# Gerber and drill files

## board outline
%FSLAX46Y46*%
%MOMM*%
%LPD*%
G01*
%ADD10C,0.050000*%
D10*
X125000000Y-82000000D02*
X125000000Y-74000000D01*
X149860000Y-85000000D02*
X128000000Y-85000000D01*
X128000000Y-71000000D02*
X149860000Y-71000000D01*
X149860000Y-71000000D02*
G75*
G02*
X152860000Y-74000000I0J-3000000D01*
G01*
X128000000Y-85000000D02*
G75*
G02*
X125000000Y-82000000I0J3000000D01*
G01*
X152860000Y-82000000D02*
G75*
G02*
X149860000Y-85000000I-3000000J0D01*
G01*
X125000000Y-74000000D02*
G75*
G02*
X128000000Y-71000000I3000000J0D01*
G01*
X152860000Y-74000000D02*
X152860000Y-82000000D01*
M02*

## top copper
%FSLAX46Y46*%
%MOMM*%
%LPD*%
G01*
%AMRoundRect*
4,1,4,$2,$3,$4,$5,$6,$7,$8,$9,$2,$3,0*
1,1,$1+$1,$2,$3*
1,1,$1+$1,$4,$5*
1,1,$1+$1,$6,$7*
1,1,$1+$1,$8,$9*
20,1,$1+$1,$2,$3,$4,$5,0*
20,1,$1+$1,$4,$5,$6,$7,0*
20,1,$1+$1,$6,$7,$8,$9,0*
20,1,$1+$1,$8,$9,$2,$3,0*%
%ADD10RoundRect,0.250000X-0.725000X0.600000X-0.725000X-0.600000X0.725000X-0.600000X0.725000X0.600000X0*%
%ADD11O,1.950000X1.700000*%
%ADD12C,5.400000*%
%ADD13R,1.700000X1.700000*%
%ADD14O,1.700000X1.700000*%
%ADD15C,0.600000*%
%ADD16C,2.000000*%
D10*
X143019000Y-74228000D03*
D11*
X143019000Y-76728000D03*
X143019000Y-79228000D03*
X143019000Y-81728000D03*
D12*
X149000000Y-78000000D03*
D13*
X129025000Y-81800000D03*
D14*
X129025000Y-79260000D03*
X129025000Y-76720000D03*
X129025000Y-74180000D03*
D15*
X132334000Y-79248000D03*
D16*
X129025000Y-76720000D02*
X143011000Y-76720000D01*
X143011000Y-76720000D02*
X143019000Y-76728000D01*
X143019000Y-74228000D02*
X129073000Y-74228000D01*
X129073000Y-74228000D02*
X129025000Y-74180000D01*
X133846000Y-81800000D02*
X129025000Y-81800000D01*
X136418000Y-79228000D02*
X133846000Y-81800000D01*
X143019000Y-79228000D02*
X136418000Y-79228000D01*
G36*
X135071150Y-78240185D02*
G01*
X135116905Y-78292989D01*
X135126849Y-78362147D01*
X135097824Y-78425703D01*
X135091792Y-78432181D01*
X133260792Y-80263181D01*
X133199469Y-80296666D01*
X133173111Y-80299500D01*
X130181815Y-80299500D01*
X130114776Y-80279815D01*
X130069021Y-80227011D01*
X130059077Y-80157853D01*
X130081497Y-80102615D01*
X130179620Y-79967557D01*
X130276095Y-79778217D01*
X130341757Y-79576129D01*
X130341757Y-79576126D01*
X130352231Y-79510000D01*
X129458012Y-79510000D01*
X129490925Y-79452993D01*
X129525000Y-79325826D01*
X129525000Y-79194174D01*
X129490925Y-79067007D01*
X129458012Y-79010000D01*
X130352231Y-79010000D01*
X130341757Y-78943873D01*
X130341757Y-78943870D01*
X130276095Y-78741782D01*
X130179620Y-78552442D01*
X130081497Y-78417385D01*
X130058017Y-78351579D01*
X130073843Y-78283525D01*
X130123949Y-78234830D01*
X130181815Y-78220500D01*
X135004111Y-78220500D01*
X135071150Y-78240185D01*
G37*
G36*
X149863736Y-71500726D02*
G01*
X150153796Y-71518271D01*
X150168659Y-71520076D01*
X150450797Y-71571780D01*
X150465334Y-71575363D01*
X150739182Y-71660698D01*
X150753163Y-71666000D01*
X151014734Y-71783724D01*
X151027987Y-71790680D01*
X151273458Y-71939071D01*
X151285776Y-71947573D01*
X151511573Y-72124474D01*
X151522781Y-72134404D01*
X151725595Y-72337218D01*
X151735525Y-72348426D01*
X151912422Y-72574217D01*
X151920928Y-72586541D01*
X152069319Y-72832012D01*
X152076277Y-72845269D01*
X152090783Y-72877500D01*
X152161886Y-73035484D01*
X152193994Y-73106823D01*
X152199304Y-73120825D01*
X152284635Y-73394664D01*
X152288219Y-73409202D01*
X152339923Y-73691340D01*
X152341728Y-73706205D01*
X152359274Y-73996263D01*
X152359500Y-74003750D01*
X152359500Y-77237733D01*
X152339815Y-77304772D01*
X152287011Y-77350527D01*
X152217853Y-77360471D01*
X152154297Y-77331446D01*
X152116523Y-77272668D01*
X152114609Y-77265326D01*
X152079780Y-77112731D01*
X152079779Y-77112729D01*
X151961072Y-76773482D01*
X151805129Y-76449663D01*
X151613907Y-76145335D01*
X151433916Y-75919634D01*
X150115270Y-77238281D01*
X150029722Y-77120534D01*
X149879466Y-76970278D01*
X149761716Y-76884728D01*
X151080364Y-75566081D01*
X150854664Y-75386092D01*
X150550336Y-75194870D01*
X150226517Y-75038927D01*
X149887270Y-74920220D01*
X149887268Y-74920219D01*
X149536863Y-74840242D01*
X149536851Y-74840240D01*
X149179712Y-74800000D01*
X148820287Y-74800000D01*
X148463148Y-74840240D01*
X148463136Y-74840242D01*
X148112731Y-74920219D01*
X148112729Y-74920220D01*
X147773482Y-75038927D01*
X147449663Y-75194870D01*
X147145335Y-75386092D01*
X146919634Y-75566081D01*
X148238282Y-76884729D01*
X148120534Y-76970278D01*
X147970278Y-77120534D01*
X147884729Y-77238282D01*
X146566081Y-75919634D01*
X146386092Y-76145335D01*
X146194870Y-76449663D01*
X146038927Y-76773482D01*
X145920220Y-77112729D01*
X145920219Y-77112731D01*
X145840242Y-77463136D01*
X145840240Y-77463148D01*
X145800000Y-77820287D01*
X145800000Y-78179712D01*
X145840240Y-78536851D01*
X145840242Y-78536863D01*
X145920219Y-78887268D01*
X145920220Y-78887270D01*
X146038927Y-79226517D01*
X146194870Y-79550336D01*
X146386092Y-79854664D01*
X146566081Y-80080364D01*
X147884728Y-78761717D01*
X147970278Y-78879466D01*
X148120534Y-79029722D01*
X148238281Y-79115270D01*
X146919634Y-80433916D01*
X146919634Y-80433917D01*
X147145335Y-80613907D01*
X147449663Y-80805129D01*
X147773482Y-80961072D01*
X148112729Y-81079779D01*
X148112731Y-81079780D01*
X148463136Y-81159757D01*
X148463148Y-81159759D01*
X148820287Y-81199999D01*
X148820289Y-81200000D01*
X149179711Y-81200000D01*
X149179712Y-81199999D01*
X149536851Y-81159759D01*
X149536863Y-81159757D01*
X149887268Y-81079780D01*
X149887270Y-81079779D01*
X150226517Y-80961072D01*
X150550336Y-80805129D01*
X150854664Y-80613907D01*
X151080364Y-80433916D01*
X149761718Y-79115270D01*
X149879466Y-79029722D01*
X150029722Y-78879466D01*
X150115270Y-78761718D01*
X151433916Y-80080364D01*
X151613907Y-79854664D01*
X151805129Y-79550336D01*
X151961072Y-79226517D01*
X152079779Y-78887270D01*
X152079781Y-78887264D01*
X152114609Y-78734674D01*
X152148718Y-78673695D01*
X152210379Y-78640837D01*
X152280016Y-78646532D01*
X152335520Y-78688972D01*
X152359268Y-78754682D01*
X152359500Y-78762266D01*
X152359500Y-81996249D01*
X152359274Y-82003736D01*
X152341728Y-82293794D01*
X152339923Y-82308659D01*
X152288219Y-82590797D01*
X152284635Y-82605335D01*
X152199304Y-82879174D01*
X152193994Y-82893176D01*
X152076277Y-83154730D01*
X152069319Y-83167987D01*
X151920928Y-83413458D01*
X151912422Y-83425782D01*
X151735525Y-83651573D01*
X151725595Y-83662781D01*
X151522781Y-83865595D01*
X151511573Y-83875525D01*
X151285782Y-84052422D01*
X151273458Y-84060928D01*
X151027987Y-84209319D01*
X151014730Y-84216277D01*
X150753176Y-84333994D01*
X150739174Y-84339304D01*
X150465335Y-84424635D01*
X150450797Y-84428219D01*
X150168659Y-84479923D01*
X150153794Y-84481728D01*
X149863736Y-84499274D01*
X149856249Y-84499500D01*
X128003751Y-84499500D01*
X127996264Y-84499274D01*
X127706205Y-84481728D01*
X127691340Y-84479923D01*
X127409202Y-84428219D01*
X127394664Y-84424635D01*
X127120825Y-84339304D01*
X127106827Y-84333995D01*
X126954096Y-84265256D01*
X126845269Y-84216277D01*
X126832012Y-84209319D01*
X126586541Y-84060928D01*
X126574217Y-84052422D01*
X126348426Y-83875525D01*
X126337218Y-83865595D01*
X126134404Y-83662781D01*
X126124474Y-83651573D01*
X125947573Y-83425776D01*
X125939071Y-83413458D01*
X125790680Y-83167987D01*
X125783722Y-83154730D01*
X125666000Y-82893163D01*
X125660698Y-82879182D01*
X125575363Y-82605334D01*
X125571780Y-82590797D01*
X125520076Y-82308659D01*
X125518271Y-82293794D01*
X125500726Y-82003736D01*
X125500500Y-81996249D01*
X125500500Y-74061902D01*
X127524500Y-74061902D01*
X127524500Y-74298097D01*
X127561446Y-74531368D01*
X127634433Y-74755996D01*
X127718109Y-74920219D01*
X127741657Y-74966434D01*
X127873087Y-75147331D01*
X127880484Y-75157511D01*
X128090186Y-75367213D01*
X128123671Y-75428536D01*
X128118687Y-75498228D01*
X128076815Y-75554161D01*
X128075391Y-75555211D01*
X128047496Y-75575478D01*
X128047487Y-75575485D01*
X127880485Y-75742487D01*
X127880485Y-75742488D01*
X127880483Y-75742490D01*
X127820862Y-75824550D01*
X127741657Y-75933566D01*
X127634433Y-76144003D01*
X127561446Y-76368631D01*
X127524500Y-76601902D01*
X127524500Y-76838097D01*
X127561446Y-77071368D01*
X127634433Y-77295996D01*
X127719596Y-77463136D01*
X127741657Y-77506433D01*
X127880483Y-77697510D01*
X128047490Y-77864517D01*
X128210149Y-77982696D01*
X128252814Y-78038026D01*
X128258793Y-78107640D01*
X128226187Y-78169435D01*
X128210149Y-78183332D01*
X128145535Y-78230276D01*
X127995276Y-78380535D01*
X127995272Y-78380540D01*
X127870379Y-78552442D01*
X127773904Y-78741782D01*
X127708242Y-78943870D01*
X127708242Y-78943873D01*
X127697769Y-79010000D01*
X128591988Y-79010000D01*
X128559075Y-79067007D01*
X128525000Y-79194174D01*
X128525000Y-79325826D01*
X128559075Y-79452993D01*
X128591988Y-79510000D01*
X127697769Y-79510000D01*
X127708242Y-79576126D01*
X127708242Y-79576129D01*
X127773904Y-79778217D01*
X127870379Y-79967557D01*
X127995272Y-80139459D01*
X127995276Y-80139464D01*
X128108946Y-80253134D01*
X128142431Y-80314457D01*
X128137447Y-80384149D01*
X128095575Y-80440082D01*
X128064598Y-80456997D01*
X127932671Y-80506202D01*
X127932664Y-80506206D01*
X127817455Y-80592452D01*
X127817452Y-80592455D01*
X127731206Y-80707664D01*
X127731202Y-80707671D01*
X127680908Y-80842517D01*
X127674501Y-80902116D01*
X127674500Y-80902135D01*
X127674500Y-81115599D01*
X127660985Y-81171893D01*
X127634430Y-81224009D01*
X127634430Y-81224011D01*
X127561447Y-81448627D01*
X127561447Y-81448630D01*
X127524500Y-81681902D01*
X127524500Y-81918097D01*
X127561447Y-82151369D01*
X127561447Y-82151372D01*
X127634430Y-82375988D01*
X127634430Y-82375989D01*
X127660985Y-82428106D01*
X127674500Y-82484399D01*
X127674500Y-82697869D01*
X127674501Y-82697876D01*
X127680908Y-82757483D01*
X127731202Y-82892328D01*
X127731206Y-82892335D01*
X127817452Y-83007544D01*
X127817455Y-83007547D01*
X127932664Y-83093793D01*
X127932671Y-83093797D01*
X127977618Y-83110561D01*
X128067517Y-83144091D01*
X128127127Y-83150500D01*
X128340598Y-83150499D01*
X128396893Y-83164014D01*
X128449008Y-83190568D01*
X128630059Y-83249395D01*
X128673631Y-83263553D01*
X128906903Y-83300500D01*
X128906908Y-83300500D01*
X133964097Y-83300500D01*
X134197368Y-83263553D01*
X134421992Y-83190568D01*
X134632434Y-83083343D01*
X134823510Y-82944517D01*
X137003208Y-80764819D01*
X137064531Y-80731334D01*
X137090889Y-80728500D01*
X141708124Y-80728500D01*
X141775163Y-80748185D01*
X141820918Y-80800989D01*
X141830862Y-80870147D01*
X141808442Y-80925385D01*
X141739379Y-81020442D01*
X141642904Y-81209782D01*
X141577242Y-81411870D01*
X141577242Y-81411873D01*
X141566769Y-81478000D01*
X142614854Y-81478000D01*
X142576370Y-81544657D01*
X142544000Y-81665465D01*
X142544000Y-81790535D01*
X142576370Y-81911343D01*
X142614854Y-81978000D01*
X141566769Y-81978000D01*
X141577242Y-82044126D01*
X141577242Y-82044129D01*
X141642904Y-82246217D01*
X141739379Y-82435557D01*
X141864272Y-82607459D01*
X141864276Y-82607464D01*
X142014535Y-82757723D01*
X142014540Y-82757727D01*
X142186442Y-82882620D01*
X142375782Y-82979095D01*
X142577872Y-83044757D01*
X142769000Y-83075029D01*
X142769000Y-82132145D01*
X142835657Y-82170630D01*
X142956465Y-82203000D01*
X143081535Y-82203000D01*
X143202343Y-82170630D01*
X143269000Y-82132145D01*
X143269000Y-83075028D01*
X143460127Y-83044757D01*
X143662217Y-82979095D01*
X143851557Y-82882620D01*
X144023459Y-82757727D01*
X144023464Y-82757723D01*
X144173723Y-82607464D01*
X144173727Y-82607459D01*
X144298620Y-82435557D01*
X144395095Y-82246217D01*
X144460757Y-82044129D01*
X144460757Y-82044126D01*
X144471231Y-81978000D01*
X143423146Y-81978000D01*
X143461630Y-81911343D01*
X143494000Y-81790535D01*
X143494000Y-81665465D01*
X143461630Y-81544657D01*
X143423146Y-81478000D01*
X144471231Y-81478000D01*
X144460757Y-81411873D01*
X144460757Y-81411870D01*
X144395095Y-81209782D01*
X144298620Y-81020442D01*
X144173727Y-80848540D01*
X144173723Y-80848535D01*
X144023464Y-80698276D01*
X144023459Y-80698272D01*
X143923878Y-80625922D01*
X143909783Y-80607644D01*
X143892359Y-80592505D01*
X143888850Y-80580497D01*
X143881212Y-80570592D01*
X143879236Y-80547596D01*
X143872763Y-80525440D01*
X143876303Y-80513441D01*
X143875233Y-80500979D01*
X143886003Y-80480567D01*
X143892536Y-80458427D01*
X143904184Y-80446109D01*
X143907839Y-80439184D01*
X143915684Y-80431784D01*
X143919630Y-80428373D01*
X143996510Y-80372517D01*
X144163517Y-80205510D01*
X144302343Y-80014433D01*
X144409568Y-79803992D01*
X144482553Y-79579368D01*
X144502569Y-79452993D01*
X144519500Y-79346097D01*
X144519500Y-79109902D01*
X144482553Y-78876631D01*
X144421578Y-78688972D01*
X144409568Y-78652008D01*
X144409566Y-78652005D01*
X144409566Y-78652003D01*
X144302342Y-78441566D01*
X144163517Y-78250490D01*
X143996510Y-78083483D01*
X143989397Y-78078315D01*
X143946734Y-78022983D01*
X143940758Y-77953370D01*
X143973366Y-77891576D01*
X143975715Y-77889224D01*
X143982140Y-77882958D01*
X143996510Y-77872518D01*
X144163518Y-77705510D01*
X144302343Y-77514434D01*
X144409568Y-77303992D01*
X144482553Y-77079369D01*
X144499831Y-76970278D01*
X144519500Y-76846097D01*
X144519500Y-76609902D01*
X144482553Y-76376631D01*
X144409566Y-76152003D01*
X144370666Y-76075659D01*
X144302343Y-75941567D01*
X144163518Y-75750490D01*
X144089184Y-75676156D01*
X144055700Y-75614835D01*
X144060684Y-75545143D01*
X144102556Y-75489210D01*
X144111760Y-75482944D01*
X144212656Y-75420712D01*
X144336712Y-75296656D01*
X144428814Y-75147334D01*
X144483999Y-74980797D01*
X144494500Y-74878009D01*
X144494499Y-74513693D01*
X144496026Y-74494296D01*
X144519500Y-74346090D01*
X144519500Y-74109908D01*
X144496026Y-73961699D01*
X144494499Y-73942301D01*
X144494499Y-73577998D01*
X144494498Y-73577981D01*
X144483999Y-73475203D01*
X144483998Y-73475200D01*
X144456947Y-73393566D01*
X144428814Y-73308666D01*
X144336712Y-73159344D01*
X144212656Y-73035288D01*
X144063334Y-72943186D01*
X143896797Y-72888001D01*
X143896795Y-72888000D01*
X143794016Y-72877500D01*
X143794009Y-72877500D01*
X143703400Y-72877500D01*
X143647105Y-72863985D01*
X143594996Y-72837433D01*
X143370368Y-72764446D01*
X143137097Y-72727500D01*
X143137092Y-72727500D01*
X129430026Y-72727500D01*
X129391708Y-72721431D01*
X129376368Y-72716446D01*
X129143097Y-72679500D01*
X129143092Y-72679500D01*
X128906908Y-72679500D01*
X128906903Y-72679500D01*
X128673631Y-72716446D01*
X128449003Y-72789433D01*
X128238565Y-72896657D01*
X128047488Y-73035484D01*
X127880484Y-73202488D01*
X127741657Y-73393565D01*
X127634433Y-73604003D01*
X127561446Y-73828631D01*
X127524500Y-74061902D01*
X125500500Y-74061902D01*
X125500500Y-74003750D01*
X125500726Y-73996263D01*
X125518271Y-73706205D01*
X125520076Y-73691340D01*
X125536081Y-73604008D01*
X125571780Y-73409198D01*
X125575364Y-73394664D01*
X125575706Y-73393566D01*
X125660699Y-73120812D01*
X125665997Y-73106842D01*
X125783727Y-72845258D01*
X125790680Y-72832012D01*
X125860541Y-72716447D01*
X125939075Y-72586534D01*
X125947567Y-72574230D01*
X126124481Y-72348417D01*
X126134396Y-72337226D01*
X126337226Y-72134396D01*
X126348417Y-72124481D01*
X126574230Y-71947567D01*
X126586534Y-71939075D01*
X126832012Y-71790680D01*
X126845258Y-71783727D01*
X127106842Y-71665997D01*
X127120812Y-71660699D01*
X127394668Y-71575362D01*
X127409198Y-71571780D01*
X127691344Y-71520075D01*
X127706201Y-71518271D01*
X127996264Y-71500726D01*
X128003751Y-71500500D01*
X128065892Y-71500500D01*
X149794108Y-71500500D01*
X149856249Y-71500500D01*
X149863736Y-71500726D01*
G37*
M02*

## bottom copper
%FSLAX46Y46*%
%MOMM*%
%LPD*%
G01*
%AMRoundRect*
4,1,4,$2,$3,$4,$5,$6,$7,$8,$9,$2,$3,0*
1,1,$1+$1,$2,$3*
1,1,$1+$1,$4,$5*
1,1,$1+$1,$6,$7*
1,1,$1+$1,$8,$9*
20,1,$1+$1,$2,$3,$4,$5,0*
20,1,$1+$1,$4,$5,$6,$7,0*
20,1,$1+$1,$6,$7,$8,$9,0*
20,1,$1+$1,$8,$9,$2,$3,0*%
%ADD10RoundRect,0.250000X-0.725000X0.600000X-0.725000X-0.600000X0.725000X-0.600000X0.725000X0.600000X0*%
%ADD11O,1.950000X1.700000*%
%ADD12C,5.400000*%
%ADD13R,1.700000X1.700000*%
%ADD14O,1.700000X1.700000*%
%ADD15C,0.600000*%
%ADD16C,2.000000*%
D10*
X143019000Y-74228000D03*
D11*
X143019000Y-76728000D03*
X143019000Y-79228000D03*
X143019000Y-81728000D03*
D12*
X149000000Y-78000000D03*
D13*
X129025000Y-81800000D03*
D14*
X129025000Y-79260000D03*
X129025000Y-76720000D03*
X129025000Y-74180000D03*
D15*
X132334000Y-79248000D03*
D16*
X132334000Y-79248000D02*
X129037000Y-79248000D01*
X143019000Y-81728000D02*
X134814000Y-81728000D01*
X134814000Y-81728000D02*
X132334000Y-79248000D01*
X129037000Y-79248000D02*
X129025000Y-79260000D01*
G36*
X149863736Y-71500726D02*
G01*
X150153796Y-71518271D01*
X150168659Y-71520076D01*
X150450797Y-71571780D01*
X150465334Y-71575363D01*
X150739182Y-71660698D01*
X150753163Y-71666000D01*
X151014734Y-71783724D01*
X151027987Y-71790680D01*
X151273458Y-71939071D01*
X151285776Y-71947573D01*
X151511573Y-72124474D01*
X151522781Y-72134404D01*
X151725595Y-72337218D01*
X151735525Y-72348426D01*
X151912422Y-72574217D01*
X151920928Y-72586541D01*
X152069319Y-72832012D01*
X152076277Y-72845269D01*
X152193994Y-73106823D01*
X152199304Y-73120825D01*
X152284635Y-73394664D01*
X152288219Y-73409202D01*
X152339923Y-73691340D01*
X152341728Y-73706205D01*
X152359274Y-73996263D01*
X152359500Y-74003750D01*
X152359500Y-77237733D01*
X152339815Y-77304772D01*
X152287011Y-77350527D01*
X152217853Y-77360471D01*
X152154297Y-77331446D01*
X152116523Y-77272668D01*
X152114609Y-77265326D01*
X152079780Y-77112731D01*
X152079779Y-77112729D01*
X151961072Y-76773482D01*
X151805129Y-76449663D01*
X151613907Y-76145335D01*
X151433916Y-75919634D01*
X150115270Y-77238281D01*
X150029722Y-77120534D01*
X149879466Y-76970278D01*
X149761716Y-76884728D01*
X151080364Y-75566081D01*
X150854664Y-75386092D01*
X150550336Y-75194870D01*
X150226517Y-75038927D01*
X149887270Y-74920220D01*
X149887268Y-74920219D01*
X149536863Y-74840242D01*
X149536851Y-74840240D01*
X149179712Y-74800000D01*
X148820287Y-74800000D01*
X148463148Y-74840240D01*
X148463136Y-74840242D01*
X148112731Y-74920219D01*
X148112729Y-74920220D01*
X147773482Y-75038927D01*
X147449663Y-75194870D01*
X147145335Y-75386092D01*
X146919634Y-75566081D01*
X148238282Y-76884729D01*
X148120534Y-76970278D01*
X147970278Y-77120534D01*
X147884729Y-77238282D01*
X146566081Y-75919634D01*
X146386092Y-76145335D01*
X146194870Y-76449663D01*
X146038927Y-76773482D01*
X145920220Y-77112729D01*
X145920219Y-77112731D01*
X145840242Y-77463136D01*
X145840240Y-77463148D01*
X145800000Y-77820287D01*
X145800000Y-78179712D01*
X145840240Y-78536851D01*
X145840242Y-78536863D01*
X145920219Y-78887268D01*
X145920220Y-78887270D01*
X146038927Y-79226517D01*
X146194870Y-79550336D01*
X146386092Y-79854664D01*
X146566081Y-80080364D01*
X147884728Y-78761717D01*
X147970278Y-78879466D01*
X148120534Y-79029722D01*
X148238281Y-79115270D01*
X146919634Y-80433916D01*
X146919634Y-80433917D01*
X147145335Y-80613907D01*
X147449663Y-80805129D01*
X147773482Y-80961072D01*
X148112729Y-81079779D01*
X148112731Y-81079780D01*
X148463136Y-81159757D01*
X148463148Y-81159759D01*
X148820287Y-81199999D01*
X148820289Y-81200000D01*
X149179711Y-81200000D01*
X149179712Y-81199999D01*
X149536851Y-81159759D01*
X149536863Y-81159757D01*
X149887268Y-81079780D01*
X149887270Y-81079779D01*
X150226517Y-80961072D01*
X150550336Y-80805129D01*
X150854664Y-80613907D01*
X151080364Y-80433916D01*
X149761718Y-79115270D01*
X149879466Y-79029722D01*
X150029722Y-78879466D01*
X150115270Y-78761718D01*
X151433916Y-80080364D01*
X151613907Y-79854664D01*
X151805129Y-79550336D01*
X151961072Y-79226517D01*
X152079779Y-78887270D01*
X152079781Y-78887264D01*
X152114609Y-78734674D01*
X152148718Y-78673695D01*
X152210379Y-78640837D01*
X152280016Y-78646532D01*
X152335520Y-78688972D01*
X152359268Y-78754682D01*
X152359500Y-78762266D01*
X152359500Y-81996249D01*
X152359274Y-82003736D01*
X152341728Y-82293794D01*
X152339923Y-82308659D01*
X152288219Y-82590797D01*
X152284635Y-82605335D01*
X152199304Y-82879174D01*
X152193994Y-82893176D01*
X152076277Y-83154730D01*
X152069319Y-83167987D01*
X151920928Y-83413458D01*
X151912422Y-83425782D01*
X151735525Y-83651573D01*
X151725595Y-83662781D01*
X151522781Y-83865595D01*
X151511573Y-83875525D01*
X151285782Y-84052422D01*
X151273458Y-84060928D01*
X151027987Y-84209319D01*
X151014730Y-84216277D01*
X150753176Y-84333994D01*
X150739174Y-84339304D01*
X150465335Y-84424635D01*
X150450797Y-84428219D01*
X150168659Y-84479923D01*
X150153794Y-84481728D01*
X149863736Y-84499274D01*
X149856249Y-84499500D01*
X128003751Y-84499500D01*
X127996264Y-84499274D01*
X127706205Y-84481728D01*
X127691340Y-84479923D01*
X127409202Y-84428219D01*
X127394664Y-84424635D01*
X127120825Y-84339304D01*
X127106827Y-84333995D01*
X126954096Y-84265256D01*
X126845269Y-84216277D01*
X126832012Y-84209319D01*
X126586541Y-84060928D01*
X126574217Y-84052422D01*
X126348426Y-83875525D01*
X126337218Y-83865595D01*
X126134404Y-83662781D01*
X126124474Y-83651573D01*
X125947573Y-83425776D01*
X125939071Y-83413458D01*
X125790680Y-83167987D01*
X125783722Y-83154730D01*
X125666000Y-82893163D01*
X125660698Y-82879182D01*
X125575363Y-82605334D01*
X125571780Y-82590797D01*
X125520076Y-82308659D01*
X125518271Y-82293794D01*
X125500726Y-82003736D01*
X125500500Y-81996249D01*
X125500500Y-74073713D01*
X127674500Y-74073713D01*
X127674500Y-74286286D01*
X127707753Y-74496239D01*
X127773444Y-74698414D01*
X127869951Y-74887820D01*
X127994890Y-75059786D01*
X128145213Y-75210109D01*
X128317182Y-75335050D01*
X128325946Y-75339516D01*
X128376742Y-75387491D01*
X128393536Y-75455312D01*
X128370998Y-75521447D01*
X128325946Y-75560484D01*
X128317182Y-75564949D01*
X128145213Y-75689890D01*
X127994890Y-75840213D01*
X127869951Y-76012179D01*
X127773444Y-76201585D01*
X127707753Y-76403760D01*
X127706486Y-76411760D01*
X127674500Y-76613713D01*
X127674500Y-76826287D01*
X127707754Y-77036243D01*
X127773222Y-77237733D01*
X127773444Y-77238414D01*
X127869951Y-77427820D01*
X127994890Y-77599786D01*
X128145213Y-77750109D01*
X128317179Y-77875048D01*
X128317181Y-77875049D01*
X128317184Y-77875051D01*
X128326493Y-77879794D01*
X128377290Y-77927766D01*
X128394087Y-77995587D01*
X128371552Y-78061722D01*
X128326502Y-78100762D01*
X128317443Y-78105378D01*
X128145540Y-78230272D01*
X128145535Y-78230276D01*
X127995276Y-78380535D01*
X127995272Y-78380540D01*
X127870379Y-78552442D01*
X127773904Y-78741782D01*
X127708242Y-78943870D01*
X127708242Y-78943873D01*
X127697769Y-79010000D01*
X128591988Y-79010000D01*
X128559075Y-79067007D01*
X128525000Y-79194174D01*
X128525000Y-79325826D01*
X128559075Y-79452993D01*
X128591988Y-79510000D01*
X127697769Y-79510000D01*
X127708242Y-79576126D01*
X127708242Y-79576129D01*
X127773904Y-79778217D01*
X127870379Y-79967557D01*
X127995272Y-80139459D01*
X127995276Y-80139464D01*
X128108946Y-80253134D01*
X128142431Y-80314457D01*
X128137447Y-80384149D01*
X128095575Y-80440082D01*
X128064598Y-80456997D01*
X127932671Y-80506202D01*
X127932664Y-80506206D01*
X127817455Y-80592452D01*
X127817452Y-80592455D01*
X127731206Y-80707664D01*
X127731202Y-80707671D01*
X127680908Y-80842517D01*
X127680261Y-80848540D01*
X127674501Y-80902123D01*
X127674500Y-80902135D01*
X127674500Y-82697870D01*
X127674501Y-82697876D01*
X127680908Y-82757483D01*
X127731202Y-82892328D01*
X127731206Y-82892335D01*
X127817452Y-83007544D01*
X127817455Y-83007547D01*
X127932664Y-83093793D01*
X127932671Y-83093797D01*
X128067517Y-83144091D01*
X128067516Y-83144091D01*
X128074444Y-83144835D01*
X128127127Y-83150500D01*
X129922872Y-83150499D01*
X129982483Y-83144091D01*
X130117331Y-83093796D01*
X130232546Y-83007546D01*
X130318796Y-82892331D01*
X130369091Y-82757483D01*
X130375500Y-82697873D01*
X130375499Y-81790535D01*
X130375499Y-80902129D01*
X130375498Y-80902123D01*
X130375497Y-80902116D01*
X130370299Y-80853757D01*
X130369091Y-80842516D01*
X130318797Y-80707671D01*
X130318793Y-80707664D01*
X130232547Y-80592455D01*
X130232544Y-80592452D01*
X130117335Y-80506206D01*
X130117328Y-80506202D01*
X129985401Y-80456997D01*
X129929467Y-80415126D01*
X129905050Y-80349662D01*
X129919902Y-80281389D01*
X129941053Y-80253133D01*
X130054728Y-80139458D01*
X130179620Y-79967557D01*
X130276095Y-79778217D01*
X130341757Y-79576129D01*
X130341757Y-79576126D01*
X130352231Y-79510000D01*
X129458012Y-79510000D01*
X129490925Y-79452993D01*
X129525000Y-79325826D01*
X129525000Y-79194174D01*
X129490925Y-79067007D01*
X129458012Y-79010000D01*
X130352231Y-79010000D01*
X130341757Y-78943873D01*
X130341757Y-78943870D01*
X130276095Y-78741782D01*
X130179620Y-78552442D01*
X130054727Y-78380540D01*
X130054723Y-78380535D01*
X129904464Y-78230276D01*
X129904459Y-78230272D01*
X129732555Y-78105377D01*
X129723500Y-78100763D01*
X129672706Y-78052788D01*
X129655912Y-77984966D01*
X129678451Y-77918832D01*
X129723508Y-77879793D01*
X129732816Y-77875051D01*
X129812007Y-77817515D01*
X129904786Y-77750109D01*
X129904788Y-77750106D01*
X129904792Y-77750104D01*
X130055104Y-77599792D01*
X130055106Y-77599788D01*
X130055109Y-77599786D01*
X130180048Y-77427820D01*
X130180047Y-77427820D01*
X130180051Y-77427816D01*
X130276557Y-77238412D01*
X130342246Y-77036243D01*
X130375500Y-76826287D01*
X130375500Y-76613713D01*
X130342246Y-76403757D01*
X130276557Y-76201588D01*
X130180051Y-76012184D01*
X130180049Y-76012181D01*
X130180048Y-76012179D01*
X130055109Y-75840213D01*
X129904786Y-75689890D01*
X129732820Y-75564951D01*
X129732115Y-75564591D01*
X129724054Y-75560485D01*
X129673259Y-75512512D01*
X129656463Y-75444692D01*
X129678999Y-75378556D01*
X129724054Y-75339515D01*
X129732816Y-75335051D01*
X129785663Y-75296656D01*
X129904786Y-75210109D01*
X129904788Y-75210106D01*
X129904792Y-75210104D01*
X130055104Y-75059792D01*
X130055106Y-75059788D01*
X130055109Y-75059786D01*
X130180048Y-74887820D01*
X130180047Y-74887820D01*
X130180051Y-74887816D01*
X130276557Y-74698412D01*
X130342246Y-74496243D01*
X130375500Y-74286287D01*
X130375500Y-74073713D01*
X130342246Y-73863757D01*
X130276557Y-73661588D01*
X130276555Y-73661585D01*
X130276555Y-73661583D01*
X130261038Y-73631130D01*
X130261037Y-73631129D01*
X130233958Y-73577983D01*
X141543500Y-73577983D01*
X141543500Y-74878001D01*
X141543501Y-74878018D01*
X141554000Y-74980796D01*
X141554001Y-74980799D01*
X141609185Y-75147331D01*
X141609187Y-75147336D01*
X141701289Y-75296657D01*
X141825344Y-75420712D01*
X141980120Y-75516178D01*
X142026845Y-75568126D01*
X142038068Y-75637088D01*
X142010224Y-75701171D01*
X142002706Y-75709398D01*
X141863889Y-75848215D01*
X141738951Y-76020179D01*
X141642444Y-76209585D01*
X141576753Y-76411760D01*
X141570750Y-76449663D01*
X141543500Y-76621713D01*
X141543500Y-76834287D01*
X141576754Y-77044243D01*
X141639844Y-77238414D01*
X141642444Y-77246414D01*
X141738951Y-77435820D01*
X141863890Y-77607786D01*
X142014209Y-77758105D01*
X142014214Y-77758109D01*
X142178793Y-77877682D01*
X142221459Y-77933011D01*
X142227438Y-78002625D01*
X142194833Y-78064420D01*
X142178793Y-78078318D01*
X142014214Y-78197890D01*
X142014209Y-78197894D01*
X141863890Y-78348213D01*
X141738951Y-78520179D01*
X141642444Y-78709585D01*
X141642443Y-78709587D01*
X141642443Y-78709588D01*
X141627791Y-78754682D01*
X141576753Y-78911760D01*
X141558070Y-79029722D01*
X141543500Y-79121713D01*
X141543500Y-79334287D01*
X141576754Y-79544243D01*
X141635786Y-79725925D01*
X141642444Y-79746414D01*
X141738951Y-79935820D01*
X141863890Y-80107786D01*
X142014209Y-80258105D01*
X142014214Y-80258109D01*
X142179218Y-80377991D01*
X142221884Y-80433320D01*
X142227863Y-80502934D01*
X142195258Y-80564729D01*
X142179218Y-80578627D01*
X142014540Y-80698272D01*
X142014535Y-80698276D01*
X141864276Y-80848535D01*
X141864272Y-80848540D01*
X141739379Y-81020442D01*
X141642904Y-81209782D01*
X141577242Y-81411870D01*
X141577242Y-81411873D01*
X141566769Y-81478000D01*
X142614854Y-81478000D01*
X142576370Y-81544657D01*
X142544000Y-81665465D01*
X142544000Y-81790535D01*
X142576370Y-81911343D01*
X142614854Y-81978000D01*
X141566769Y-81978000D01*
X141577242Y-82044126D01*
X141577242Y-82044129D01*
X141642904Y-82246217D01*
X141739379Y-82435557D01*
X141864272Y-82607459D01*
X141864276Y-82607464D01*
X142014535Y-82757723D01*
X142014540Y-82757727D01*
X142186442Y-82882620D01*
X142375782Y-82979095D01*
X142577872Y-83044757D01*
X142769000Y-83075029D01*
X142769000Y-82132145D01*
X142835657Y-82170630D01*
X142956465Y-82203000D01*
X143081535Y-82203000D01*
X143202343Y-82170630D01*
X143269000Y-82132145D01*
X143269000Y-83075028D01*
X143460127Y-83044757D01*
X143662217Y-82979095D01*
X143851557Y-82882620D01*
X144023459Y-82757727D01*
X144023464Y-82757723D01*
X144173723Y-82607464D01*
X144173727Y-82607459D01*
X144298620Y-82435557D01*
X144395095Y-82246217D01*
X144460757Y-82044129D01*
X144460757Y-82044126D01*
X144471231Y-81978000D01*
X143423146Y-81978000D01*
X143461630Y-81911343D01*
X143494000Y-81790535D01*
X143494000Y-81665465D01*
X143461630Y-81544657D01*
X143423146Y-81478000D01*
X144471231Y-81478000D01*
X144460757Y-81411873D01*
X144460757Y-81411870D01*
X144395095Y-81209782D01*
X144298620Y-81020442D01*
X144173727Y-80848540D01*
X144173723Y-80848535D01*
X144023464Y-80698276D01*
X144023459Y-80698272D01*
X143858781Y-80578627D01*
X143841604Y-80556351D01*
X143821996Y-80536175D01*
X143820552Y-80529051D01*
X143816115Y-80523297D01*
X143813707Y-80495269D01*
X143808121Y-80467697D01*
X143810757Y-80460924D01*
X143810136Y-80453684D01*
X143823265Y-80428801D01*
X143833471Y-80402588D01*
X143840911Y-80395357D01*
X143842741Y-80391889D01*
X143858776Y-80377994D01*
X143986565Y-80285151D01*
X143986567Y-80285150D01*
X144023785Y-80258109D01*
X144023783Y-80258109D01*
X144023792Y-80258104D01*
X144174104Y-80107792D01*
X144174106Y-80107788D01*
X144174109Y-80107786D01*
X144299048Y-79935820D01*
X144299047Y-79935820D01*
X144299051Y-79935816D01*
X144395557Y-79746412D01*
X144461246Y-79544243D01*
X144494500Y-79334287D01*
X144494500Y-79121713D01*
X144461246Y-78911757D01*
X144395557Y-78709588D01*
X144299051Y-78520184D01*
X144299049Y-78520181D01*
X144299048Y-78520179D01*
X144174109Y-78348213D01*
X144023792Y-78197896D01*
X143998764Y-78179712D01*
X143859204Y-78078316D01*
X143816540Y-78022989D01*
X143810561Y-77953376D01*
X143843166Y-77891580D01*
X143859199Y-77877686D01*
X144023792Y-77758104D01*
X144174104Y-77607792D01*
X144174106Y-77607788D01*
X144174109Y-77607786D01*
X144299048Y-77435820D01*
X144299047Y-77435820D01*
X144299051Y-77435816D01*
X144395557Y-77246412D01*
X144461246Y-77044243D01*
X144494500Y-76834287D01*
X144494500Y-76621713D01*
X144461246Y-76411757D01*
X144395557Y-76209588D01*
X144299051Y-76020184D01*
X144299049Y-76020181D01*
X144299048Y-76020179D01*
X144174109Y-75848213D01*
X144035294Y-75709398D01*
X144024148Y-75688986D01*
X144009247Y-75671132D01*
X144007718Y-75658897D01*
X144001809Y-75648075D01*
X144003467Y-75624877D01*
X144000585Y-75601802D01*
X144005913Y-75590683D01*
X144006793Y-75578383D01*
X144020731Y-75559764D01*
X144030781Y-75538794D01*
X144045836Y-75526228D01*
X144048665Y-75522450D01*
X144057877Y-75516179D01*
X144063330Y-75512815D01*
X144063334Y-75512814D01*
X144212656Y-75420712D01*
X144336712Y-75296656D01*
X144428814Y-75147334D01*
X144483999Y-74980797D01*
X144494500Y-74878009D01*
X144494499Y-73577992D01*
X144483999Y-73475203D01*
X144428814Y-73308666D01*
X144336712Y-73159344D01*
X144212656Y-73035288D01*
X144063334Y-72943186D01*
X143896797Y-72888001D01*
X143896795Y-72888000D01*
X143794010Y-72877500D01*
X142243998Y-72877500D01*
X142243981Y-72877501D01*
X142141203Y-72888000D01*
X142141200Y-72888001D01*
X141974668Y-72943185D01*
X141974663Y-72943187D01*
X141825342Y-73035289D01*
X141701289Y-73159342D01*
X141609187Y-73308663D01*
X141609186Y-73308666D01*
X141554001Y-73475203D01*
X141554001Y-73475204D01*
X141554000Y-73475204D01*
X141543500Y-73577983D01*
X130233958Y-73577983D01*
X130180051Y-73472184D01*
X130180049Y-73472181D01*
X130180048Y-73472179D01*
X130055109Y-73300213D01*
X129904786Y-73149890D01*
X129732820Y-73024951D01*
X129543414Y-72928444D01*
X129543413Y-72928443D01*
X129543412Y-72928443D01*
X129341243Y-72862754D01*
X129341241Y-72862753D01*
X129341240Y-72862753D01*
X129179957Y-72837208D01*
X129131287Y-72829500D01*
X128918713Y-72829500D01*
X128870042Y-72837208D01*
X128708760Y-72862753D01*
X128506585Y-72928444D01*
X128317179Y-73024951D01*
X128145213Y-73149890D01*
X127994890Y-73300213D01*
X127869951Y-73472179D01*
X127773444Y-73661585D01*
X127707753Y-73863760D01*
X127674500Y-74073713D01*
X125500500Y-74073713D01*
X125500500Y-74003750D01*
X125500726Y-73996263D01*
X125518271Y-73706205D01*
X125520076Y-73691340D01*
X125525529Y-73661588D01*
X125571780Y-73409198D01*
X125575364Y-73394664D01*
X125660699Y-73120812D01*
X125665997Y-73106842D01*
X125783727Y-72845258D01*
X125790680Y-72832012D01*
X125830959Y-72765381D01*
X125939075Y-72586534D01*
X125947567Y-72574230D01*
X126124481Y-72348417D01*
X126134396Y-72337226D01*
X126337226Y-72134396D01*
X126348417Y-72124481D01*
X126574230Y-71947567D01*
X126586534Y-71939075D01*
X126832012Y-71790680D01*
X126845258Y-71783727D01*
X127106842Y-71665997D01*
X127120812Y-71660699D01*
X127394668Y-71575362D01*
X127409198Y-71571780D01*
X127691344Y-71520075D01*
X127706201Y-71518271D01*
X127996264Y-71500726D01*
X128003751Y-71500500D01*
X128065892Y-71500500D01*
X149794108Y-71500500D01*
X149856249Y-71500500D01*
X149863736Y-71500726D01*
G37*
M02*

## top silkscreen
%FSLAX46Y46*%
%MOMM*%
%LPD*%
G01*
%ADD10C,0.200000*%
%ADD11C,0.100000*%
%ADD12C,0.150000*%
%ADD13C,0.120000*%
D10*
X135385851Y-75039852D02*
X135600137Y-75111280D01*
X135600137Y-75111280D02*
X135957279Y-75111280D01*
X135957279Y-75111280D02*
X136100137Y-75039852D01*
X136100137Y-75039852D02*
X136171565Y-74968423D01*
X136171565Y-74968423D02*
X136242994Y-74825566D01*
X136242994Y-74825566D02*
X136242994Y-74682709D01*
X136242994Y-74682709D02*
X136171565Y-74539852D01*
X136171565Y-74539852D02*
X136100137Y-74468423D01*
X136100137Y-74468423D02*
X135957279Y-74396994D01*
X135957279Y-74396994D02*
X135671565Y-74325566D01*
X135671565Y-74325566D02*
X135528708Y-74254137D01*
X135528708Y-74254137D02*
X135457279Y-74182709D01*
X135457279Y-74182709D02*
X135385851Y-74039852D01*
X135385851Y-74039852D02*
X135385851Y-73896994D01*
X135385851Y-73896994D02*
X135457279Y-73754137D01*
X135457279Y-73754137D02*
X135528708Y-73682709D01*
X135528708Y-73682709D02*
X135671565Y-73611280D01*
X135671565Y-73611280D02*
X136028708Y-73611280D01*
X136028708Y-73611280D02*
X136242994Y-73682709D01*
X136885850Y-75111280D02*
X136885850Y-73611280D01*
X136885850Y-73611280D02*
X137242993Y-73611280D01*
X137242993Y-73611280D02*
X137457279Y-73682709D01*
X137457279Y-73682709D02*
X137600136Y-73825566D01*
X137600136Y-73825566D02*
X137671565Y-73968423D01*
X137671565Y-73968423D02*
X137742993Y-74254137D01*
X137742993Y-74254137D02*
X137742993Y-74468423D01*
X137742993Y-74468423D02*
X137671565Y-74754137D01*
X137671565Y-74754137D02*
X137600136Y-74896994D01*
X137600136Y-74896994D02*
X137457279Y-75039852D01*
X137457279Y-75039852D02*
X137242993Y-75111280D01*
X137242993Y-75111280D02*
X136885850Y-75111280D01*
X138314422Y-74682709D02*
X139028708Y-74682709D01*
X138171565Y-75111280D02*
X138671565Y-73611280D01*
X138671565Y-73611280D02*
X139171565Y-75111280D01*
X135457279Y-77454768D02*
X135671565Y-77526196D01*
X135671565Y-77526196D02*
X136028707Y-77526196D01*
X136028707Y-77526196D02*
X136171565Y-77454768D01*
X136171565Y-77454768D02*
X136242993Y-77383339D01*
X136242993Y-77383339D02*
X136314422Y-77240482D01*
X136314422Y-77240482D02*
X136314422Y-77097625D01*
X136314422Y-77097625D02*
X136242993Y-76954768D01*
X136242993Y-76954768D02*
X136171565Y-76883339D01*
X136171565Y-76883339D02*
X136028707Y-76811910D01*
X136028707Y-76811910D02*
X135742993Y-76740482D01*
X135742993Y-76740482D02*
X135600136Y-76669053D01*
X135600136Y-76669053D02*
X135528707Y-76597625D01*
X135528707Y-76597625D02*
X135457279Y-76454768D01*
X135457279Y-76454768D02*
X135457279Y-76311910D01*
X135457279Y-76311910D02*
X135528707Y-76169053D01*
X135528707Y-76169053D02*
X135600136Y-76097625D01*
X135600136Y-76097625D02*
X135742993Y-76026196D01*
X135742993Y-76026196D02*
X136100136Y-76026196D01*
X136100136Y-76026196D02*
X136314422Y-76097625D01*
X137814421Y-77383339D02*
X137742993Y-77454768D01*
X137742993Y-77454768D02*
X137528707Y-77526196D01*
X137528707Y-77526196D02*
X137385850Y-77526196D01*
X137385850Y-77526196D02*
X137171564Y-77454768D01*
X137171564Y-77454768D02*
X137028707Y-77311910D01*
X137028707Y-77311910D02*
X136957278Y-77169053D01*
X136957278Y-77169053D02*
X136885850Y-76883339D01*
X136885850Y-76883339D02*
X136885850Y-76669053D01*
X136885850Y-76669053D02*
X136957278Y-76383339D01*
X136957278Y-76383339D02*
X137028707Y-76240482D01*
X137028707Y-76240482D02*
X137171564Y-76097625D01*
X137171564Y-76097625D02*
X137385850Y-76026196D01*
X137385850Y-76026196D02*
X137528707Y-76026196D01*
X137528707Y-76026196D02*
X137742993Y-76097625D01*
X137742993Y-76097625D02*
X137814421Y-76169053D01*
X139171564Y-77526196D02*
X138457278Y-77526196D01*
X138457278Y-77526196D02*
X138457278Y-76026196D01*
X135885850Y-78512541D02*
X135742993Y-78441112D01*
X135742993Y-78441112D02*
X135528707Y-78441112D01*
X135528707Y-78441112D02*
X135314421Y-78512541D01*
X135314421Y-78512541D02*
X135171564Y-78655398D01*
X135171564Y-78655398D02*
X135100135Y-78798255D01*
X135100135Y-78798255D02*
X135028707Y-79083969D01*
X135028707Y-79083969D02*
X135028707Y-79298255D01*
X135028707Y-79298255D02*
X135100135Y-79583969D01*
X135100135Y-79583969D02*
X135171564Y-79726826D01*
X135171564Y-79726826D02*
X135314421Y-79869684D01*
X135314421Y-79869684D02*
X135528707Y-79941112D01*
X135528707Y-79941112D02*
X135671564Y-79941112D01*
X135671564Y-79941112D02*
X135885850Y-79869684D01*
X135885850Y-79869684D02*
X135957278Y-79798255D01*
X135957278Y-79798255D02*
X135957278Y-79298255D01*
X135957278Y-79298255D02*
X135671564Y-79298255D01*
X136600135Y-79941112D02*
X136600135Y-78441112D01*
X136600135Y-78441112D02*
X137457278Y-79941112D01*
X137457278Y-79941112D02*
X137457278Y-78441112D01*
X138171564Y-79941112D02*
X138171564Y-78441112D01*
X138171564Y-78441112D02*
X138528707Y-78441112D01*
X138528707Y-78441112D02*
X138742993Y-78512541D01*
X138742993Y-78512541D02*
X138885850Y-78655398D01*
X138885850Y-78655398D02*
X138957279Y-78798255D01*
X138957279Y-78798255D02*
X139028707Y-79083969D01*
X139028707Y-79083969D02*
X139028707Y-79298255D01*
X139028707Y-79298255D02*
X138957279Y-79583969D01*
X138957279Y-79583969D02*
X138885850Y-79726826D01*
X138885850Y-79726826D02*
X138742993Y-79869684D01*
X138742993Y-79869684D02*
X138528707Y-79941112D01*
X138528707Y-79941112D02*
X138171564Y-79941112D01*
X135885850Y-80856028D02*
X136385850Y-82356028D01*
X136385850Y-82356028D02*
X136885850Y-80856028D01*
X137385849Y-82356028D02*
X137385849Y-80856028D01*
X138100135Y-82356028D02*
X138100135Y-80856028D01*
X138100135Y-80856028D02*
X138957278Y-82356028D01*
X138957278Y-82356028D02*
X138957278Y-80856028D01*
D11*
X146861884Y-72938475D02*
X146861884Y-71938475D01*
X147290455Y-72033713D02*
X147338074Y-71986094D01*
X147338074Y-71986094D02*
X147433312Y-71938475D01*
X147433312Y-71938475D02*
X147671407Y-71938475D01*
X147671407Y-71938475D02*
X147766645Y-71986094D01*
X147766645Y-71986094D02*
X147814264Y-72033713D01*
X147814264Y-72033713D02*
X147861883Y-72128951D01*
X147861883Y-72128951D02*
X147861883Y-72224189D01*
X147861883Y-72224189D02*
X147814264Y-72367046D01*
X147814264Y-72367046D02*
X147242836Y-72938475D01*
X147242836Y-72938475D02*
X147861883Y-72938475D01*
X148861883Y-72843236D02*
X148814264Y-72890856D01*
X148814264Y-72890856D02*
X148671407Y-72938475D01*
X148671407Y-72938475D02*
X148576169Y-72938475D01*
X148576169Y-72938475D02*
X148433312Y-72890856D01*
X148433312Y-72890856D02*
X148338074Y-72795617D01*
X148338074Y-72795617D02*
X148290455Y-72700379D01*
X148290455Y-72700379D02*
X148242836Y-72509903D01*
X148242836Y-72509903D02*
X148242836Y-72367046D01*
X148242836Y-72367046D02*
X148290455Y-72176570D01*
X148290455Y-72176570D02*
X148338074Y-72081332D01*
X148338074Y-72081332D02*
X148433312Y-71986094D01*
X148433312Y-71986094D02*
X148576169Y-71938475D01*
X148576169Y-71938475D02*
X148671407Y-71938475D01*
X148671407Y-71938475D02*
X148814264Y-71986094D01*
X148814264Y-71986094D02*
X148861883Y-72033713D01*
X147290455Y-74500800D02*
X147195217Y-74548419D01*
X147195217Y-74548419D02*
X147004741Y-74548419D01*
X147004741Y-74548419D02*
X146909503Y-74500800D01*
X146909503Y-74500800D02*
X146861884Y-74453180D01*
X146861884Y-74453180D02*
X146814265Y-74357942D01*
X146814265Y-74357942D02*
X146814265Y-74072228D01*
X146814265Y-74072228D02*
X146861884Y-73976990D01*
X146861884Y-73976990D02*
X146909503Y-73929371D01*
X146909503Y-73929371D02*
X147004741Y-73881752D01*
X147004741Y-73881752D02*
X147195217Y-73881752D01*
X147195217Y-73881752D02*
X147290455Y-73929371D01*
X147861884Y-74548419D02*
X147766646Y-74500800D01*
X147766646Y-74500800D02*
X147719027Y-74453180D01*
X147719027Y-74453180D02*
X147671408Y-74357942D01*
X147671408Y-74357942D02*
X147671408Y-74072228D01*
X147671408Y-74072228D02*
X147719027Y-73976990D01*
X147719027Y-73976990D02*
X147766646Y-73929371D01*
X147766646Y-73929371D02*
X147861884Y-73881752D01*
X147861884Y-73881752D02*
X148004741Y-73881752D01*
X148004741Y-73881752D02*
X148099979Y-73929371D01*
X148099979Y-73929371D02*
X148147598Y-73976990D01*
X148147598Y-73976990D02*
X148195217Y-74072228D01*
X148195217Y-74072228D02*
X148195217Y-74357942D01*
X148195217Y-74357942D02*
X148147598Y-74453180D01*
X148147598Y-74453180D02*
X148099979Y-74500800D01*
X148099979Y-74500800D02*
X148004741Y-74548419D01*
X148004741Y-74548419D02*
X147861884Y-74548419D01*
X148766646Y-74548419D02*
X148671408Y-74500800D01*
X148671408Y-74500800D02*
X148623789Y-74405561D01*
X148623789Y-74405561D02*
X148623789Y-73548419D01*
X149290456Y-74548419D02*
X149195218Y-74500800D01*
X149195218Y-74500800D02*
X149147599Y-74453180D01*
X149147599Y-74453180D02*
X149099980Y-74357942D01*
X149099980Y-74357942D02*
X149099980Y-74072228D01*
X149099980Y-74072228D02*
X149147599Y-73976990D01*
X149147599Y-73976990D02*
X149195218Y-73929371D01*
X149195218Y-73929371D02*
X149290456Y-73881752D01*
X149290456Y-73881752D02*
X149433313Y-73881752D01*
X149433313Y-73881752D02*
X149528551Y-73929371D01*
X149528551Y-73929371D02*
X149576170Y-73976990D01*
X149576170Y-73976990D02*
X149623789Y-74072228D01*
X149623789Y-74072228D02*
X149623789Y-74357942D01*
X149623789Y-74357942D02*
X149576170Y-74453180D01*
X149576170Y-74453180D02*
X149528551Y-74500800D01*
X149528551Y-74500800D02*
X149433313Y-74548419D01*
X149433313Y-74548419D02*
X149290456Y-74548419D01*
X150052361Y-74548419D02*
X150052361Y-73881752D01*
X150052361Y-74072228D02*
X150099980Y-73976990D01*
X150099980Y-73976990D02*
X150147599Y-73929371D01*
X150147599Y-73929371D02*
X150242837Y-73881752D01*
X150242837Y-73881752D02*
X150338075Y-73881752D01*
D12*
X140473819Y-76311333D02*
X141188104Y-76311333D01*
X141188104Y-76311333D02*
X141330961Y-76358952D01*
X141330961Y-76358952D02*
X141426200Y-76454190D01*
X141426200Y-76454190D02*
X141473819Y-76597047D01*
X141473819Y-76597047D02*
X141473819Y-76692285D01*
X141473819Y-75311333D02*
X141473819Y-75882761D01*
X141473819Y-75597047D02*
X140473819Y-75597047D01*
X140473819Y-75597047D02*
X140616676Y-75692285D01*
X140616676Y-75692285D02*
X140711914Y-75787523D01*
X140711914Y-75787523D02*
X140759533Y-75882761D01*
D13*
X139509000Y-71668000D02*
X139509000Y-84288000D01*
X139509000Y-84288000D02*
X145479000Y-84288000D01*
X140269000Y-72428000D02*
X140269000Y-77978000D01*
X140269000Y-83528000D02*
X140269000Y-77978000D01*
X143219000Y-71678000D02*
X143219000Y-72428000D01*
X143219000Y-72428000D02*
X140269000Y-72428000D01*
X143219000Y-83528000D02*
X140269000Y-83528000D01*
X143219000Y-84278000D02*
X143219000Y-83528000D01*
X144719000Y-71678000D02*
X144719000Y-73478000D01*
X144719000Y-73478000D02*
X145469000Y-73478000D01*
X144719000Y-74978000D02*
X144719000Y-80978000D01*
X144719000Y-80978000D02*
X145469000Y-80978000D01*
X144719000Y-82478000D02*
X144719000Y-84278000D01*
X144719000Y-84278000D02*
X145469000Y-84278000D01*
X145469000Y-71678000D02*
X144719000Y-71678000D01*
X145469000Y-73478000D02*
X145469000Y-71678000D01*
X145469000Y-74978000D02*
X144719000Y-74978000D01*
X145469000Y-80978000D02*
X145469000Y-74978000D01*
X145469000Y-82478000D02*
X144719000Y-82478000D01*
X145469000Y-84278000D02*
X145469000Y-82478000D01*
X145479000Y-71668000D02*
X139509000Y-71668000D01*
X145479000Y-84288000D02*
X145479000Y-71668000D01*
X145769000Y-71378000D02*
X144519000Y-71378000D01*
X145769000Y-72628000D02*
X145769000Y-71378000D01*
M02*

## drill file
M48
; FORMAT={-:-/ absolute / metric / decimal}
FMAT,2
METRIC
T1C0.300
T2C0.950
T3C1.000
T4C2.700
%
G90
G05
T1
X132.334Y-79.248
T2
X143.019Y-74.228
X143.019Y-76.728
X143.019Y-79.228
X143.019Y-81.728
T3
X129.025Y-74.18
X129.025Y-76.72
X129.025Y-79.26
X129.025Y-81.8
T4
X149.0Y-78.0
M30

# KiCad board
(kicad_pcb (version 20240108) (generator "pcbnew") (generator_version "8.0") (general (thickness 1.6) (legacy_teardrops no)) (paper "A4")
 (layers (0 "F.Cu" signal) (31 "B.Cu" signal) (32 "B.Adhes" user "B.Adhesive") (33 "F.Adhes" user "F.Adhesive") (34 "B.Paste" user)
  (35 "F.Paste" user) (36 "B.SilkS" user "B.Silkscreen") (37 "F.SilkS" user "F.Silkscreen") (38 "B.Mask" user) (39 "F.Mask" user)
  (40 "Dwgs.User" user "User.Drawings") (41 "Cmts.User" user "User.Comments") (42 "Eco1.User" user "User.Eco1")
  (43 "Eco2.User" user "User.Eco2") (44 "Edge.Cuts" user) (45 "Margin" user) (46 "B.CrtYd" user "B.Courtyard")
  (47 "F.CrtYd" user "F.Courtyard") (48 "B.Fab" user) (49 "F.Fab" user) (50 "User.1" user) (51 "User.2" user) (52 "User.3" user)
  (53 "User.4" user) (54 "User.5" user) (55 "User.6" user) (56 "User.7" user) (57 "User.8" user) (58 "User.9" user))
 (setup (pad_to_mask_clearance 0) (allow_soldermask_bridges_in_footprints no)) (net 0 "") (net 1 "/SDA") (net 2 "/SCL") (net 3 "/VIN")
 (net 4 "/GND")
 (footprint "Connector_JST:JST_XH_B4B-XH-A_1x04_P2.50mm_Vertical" (layer "F.Cu") (at 143.019 74.228 -90)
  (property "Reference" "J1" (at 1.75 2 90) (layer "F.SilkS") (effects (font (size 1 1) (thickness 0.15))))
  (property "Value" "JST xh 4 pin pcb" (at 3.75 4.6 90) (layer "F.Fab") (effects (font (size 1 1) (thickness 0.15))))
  (fp_line (start -2.56 3.51) (end 10.06 3.51) (stroke (width 0.12) (type solid)) (layer "F.SilkS"))
  (fp_line (start 10.06 3.51) (end 10.06 -2.46) (stroke (width 0.12) (type solid)) (layer "F.SilkS"))
  (fp_line (start -1.8 2.75) (end 3.75 2.75) (stroke (width 0.12) (type solid)) (layer "F.SilkS"))
  (fp_line (start 9.3 2.75) (end 3.75 2.75) (stroke (width 0.12) (type solid)) (layer "F.SilkS"))
  (fp_line (start -2.55 -0.2) (end -1.8 -0.2) (stroke (width 0.12) (type solid)) (layer "F.SilkS"))
  (fp_line (start -1.8 -0.2) (end -1.8 2.75) (stroke (width 0.12) (type solid)) (layer "F.SilkS"))
  (fp_line (start 9.3 -0.2) (end 9.3 2.75) (stroke (width 0.12) (type solid)) (layer "F.SilkS"))
  (fp_line (start 10.05 -0.2) (end 9.3 -0.2) (stroke (width 0.12) (type solid)) (layer "F.SilkS"))
  (fp_line (start -2.55 -1.7) (end -0.75 -1.7) (stroke (width 0.12) (type solid)) (layer "F.SilkS"))
  (fp_line (start -0.75 -1.7) (end -0.75 -2.45) (stroke (width 0.12) (type solid)) (layer "F.SilkS"))
  (fp_line (start 0.75 -1.7) (end 6.75 -1.7) (stroke (width 0.12) (type solid)) (layer "F.SilkS"))
  (fp_line (start 6.75 -1.7) (end 6.75 -2.45) (stroke (width 0.12) (type solid)) (layer "F.SilkS"))
  (fp_line (start 8.25 -1.7) (end 10.05 -1.7) (stroke (width 0.12) (type solid)) (layer "F.SilkS"))
  (fp_line (start 10.05 -1.7) (end 10.05 -2.45) (stroke (width 0.12) (type solid)) (layer "F.SilkS"))
  (fp_line (start -2.55 -2.45) (end -2.55 -1.7) (stroke (width 0.12) (type solid)) (layer "F.SilkS"))
  (fp_line (start -0.75 -2.45) (end -2.55 -2.45) (stroke (width 0.12) (type solid)) (layer "F.SilkS"))
  (fp_line (start 0.75 -2.45) (end 0.75 -1.7) (stroke (width 0.12) (type solid)) (layer "F.SilkS"))
  (fp_line (start 6.75 -2.45) (end 0.75 -2.45) (stroke (width 0.12) (type solid)) (layer "F.SilkS"))
  (fp_line (start 8.25 -2.45) (end 8.25 -1.7) (stroke (width 0.12) (type solid)) (layer "F.SilkS"))
  (fp_line (start 10.05 -2.45) (end 8.25 -2.45) (stroke (width 0.12) (type solid)) (layer "F.SilkS"))
  (fp_line (start -2.56 -2.46) (end -2.56 3.51) (stroke (width 0.12) (type solid)) (layer "F.SilkS"))
  (fp_line (start 10.06 -2.46) (end -2.56 -2.46) (stroke (width 0.12) (type solid)) (layer "F.SilkS"))
  (fp_line (start -2.85 -2.75) (end -2.85 -1.5) (stroke (width 0.12) (type solid)) (layer "F.SilkS"))
  (fp_line (start -1.6 -2.75) (end -2.85 -2.75) (stroke (width 0.12) (type solid)) (layer "F.SilkS"))
  (pad "1" thru_hole roundrect (at 0 0 270) (size 1.7 1.95) (drill 0.95) (layers "*.Cu" "*.Mask") (remove_unused_layers no)
   (roundrect_rratio 0.147059) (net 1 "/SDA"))
  (pad "2" thru_hole oval (at 2.5 0 270) (size 1.7 1.95) (drill 0.95) (layers "*.Cu" "*.Mask") (remove_unused_layers no) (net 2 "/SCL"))
  (pad "3" thru_hole oval (at 5 0 270) (size 1.7 1.95) (drill 0.95) (layers "*.Cu" "*.Mask") (remove_unused_layers no) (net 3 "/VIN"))
  (pad "4" thru_hole oval (at 7.5 0 270) (size 1.7 1.95) (drill 0.95) (layers "*.Cu" "*.Mask") (remove_unused_layers no) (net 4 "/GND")))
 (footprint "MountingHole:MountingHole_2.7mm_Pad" (layer "F.Cu") (at 149 78)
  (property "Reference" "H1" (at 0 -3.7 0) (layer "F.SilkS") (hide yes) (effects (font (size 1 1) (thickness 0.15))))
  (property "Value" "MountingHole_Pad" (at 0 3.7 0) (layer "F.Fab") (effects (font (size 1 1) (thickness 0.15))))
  (pad "1" thru_hole circle (at 0 0) (size 5.4 5.4) (drill 2.7) (layers "*.Cu" "*.Mask") (remove_unused_layers no) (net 4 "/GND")))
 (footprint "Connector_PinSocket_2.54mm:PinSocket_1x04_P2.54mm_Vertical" (layer "B.Cu") (at 129.025 81.8)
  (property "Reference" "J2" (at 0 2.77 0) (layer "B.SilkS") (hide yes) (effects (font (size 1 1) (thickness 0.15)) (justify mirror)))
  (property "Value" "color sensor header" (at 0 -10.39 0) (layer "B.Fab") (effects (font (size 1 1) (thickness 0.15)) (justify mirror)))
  (pad "1" thru_hole rect (at 0 0) (size 1.7 1.7) (drill 1) (layers "*.Cu" "*.Mask") (remove_unused_layers no) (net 3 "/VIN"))
  (pad "2" thru_hole oval (at 0 -2.54) (size 1.7 1.7) (drill 1) (layers "*.Cu" "*.Mask") (remove_unused_layers no) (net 4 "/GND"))
  (pad "3" thru_hole oval (at 0 -5.08) (size 1.7 1.7) (drill 1) (layers "*.Cu" "*.Mask") (remove_unused_layers no) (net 2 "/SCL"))
  (pad "4" thru_hole oval (at 0 -7.62) (size 1.7 1.7) (drill 1) (layers "*.Cu" "*.Mask") (remove_unused_layers no) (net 1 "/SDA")))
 (gr_line (start 125 82) (end 125 74) (stroke (width 0.05) (type default)) (layer "Edge.Cuts"))
 (gr_line (start 149.86 85) (end 128 85) (stroke (width 0.05) (type default)) (layer "Edge.Cuts"))
 (gr_line (start 128 71) (end 149.86 71) (stroke (width 0.05) (type default)) (layer "Edge.Cuts"))
 (gr_arc (start 149.86 71) (mid 151.98132 71.87868) (end 152.86 74) (stroke (width 0.05) (type default)) (layer "Edge.Cuts"))
 (gr_arc (start 128 85) (mid 125.87868 84.12132) (end 125 82) (stroke (width 0.05) (type default)) (layer "Edge.Cuts"))
 (gr_arc (start 152.86 82) (mid 151.98132 84.12132) (end 149.86 85) (stroke (width 0.05) (type default)) (layer "Edge.Cuts"))
 (gr_arc (start 125 74) (mid 125.87868 71.87868) (end 128 71) (stroke (width 0.05) (type default)) (layer "Edge.Cuts"))
 (gr_line (start 152.86 74) (end 152.86 82) (stroke (width 0.05) (type default)) (layer "Edge.Cuts"))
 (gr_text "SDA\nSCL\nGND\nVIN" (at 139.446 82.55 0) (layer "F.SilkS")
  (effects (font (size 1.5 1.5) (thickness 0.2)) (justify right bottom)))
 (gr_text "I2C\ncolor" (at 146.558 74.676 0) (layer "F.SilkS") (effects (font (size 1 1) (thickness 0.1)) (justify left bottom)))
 (segment (start 129.025 76.72) (end 143.011 76.72) (width 2) (layer "F.Cu") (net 2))
 (segment (start 143.011 76.72) (end 143.019 76.728) (width 2) (layer "F.Cu") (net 2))
 (segment (start 143.019 74.228) (end 129.073 74.228) (width 2) (layer "F.Cu") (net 1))
 (segment (start 129.073 74.228) (end 129.025 74.18) (width 2) (layer "F.Cu") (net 1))
 (via (at 132.334 79.248) (size 0.6) (drill 0.3) (layers "F.Cu" "B.Cu") (free yes) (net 4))
 (segment (start 132.334 79.248) (end 129.037 79.248) (width 2) (layer "B.Cu") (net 4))
 (segment (start 143.019 81.728) (end 134.814 81.728) (width 2) (layer "B.Cu") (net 4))
 (segment (start 134.814 81.728) (end 132.334 79.248) (width 2) (layer "B.Cu") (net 4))
 (segment (start 129.037 79.248) (end 129.025 79.26) (width 2) (layer "B.Cu") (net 4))
 (segment (start 133.846 81.8) (end 129.025 81.8) (width 2) (layer "F.Cu") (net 3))
 (segment (start 136.418 79.228) (end 133.846 81.8) (width 2) (layer "F.Cu") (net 3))
 (segment (start 143.019 79.228) (end 136.418 79.228) (width 2) (layer "F.Cu") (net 3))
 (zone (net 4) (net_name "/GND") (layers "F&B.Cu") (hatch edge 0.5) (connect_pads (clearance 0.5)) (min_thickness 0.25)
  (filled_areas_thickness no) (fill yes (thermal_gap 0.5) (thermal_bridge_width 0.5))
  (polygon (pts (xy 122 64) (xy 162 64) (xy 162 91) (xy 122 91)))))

